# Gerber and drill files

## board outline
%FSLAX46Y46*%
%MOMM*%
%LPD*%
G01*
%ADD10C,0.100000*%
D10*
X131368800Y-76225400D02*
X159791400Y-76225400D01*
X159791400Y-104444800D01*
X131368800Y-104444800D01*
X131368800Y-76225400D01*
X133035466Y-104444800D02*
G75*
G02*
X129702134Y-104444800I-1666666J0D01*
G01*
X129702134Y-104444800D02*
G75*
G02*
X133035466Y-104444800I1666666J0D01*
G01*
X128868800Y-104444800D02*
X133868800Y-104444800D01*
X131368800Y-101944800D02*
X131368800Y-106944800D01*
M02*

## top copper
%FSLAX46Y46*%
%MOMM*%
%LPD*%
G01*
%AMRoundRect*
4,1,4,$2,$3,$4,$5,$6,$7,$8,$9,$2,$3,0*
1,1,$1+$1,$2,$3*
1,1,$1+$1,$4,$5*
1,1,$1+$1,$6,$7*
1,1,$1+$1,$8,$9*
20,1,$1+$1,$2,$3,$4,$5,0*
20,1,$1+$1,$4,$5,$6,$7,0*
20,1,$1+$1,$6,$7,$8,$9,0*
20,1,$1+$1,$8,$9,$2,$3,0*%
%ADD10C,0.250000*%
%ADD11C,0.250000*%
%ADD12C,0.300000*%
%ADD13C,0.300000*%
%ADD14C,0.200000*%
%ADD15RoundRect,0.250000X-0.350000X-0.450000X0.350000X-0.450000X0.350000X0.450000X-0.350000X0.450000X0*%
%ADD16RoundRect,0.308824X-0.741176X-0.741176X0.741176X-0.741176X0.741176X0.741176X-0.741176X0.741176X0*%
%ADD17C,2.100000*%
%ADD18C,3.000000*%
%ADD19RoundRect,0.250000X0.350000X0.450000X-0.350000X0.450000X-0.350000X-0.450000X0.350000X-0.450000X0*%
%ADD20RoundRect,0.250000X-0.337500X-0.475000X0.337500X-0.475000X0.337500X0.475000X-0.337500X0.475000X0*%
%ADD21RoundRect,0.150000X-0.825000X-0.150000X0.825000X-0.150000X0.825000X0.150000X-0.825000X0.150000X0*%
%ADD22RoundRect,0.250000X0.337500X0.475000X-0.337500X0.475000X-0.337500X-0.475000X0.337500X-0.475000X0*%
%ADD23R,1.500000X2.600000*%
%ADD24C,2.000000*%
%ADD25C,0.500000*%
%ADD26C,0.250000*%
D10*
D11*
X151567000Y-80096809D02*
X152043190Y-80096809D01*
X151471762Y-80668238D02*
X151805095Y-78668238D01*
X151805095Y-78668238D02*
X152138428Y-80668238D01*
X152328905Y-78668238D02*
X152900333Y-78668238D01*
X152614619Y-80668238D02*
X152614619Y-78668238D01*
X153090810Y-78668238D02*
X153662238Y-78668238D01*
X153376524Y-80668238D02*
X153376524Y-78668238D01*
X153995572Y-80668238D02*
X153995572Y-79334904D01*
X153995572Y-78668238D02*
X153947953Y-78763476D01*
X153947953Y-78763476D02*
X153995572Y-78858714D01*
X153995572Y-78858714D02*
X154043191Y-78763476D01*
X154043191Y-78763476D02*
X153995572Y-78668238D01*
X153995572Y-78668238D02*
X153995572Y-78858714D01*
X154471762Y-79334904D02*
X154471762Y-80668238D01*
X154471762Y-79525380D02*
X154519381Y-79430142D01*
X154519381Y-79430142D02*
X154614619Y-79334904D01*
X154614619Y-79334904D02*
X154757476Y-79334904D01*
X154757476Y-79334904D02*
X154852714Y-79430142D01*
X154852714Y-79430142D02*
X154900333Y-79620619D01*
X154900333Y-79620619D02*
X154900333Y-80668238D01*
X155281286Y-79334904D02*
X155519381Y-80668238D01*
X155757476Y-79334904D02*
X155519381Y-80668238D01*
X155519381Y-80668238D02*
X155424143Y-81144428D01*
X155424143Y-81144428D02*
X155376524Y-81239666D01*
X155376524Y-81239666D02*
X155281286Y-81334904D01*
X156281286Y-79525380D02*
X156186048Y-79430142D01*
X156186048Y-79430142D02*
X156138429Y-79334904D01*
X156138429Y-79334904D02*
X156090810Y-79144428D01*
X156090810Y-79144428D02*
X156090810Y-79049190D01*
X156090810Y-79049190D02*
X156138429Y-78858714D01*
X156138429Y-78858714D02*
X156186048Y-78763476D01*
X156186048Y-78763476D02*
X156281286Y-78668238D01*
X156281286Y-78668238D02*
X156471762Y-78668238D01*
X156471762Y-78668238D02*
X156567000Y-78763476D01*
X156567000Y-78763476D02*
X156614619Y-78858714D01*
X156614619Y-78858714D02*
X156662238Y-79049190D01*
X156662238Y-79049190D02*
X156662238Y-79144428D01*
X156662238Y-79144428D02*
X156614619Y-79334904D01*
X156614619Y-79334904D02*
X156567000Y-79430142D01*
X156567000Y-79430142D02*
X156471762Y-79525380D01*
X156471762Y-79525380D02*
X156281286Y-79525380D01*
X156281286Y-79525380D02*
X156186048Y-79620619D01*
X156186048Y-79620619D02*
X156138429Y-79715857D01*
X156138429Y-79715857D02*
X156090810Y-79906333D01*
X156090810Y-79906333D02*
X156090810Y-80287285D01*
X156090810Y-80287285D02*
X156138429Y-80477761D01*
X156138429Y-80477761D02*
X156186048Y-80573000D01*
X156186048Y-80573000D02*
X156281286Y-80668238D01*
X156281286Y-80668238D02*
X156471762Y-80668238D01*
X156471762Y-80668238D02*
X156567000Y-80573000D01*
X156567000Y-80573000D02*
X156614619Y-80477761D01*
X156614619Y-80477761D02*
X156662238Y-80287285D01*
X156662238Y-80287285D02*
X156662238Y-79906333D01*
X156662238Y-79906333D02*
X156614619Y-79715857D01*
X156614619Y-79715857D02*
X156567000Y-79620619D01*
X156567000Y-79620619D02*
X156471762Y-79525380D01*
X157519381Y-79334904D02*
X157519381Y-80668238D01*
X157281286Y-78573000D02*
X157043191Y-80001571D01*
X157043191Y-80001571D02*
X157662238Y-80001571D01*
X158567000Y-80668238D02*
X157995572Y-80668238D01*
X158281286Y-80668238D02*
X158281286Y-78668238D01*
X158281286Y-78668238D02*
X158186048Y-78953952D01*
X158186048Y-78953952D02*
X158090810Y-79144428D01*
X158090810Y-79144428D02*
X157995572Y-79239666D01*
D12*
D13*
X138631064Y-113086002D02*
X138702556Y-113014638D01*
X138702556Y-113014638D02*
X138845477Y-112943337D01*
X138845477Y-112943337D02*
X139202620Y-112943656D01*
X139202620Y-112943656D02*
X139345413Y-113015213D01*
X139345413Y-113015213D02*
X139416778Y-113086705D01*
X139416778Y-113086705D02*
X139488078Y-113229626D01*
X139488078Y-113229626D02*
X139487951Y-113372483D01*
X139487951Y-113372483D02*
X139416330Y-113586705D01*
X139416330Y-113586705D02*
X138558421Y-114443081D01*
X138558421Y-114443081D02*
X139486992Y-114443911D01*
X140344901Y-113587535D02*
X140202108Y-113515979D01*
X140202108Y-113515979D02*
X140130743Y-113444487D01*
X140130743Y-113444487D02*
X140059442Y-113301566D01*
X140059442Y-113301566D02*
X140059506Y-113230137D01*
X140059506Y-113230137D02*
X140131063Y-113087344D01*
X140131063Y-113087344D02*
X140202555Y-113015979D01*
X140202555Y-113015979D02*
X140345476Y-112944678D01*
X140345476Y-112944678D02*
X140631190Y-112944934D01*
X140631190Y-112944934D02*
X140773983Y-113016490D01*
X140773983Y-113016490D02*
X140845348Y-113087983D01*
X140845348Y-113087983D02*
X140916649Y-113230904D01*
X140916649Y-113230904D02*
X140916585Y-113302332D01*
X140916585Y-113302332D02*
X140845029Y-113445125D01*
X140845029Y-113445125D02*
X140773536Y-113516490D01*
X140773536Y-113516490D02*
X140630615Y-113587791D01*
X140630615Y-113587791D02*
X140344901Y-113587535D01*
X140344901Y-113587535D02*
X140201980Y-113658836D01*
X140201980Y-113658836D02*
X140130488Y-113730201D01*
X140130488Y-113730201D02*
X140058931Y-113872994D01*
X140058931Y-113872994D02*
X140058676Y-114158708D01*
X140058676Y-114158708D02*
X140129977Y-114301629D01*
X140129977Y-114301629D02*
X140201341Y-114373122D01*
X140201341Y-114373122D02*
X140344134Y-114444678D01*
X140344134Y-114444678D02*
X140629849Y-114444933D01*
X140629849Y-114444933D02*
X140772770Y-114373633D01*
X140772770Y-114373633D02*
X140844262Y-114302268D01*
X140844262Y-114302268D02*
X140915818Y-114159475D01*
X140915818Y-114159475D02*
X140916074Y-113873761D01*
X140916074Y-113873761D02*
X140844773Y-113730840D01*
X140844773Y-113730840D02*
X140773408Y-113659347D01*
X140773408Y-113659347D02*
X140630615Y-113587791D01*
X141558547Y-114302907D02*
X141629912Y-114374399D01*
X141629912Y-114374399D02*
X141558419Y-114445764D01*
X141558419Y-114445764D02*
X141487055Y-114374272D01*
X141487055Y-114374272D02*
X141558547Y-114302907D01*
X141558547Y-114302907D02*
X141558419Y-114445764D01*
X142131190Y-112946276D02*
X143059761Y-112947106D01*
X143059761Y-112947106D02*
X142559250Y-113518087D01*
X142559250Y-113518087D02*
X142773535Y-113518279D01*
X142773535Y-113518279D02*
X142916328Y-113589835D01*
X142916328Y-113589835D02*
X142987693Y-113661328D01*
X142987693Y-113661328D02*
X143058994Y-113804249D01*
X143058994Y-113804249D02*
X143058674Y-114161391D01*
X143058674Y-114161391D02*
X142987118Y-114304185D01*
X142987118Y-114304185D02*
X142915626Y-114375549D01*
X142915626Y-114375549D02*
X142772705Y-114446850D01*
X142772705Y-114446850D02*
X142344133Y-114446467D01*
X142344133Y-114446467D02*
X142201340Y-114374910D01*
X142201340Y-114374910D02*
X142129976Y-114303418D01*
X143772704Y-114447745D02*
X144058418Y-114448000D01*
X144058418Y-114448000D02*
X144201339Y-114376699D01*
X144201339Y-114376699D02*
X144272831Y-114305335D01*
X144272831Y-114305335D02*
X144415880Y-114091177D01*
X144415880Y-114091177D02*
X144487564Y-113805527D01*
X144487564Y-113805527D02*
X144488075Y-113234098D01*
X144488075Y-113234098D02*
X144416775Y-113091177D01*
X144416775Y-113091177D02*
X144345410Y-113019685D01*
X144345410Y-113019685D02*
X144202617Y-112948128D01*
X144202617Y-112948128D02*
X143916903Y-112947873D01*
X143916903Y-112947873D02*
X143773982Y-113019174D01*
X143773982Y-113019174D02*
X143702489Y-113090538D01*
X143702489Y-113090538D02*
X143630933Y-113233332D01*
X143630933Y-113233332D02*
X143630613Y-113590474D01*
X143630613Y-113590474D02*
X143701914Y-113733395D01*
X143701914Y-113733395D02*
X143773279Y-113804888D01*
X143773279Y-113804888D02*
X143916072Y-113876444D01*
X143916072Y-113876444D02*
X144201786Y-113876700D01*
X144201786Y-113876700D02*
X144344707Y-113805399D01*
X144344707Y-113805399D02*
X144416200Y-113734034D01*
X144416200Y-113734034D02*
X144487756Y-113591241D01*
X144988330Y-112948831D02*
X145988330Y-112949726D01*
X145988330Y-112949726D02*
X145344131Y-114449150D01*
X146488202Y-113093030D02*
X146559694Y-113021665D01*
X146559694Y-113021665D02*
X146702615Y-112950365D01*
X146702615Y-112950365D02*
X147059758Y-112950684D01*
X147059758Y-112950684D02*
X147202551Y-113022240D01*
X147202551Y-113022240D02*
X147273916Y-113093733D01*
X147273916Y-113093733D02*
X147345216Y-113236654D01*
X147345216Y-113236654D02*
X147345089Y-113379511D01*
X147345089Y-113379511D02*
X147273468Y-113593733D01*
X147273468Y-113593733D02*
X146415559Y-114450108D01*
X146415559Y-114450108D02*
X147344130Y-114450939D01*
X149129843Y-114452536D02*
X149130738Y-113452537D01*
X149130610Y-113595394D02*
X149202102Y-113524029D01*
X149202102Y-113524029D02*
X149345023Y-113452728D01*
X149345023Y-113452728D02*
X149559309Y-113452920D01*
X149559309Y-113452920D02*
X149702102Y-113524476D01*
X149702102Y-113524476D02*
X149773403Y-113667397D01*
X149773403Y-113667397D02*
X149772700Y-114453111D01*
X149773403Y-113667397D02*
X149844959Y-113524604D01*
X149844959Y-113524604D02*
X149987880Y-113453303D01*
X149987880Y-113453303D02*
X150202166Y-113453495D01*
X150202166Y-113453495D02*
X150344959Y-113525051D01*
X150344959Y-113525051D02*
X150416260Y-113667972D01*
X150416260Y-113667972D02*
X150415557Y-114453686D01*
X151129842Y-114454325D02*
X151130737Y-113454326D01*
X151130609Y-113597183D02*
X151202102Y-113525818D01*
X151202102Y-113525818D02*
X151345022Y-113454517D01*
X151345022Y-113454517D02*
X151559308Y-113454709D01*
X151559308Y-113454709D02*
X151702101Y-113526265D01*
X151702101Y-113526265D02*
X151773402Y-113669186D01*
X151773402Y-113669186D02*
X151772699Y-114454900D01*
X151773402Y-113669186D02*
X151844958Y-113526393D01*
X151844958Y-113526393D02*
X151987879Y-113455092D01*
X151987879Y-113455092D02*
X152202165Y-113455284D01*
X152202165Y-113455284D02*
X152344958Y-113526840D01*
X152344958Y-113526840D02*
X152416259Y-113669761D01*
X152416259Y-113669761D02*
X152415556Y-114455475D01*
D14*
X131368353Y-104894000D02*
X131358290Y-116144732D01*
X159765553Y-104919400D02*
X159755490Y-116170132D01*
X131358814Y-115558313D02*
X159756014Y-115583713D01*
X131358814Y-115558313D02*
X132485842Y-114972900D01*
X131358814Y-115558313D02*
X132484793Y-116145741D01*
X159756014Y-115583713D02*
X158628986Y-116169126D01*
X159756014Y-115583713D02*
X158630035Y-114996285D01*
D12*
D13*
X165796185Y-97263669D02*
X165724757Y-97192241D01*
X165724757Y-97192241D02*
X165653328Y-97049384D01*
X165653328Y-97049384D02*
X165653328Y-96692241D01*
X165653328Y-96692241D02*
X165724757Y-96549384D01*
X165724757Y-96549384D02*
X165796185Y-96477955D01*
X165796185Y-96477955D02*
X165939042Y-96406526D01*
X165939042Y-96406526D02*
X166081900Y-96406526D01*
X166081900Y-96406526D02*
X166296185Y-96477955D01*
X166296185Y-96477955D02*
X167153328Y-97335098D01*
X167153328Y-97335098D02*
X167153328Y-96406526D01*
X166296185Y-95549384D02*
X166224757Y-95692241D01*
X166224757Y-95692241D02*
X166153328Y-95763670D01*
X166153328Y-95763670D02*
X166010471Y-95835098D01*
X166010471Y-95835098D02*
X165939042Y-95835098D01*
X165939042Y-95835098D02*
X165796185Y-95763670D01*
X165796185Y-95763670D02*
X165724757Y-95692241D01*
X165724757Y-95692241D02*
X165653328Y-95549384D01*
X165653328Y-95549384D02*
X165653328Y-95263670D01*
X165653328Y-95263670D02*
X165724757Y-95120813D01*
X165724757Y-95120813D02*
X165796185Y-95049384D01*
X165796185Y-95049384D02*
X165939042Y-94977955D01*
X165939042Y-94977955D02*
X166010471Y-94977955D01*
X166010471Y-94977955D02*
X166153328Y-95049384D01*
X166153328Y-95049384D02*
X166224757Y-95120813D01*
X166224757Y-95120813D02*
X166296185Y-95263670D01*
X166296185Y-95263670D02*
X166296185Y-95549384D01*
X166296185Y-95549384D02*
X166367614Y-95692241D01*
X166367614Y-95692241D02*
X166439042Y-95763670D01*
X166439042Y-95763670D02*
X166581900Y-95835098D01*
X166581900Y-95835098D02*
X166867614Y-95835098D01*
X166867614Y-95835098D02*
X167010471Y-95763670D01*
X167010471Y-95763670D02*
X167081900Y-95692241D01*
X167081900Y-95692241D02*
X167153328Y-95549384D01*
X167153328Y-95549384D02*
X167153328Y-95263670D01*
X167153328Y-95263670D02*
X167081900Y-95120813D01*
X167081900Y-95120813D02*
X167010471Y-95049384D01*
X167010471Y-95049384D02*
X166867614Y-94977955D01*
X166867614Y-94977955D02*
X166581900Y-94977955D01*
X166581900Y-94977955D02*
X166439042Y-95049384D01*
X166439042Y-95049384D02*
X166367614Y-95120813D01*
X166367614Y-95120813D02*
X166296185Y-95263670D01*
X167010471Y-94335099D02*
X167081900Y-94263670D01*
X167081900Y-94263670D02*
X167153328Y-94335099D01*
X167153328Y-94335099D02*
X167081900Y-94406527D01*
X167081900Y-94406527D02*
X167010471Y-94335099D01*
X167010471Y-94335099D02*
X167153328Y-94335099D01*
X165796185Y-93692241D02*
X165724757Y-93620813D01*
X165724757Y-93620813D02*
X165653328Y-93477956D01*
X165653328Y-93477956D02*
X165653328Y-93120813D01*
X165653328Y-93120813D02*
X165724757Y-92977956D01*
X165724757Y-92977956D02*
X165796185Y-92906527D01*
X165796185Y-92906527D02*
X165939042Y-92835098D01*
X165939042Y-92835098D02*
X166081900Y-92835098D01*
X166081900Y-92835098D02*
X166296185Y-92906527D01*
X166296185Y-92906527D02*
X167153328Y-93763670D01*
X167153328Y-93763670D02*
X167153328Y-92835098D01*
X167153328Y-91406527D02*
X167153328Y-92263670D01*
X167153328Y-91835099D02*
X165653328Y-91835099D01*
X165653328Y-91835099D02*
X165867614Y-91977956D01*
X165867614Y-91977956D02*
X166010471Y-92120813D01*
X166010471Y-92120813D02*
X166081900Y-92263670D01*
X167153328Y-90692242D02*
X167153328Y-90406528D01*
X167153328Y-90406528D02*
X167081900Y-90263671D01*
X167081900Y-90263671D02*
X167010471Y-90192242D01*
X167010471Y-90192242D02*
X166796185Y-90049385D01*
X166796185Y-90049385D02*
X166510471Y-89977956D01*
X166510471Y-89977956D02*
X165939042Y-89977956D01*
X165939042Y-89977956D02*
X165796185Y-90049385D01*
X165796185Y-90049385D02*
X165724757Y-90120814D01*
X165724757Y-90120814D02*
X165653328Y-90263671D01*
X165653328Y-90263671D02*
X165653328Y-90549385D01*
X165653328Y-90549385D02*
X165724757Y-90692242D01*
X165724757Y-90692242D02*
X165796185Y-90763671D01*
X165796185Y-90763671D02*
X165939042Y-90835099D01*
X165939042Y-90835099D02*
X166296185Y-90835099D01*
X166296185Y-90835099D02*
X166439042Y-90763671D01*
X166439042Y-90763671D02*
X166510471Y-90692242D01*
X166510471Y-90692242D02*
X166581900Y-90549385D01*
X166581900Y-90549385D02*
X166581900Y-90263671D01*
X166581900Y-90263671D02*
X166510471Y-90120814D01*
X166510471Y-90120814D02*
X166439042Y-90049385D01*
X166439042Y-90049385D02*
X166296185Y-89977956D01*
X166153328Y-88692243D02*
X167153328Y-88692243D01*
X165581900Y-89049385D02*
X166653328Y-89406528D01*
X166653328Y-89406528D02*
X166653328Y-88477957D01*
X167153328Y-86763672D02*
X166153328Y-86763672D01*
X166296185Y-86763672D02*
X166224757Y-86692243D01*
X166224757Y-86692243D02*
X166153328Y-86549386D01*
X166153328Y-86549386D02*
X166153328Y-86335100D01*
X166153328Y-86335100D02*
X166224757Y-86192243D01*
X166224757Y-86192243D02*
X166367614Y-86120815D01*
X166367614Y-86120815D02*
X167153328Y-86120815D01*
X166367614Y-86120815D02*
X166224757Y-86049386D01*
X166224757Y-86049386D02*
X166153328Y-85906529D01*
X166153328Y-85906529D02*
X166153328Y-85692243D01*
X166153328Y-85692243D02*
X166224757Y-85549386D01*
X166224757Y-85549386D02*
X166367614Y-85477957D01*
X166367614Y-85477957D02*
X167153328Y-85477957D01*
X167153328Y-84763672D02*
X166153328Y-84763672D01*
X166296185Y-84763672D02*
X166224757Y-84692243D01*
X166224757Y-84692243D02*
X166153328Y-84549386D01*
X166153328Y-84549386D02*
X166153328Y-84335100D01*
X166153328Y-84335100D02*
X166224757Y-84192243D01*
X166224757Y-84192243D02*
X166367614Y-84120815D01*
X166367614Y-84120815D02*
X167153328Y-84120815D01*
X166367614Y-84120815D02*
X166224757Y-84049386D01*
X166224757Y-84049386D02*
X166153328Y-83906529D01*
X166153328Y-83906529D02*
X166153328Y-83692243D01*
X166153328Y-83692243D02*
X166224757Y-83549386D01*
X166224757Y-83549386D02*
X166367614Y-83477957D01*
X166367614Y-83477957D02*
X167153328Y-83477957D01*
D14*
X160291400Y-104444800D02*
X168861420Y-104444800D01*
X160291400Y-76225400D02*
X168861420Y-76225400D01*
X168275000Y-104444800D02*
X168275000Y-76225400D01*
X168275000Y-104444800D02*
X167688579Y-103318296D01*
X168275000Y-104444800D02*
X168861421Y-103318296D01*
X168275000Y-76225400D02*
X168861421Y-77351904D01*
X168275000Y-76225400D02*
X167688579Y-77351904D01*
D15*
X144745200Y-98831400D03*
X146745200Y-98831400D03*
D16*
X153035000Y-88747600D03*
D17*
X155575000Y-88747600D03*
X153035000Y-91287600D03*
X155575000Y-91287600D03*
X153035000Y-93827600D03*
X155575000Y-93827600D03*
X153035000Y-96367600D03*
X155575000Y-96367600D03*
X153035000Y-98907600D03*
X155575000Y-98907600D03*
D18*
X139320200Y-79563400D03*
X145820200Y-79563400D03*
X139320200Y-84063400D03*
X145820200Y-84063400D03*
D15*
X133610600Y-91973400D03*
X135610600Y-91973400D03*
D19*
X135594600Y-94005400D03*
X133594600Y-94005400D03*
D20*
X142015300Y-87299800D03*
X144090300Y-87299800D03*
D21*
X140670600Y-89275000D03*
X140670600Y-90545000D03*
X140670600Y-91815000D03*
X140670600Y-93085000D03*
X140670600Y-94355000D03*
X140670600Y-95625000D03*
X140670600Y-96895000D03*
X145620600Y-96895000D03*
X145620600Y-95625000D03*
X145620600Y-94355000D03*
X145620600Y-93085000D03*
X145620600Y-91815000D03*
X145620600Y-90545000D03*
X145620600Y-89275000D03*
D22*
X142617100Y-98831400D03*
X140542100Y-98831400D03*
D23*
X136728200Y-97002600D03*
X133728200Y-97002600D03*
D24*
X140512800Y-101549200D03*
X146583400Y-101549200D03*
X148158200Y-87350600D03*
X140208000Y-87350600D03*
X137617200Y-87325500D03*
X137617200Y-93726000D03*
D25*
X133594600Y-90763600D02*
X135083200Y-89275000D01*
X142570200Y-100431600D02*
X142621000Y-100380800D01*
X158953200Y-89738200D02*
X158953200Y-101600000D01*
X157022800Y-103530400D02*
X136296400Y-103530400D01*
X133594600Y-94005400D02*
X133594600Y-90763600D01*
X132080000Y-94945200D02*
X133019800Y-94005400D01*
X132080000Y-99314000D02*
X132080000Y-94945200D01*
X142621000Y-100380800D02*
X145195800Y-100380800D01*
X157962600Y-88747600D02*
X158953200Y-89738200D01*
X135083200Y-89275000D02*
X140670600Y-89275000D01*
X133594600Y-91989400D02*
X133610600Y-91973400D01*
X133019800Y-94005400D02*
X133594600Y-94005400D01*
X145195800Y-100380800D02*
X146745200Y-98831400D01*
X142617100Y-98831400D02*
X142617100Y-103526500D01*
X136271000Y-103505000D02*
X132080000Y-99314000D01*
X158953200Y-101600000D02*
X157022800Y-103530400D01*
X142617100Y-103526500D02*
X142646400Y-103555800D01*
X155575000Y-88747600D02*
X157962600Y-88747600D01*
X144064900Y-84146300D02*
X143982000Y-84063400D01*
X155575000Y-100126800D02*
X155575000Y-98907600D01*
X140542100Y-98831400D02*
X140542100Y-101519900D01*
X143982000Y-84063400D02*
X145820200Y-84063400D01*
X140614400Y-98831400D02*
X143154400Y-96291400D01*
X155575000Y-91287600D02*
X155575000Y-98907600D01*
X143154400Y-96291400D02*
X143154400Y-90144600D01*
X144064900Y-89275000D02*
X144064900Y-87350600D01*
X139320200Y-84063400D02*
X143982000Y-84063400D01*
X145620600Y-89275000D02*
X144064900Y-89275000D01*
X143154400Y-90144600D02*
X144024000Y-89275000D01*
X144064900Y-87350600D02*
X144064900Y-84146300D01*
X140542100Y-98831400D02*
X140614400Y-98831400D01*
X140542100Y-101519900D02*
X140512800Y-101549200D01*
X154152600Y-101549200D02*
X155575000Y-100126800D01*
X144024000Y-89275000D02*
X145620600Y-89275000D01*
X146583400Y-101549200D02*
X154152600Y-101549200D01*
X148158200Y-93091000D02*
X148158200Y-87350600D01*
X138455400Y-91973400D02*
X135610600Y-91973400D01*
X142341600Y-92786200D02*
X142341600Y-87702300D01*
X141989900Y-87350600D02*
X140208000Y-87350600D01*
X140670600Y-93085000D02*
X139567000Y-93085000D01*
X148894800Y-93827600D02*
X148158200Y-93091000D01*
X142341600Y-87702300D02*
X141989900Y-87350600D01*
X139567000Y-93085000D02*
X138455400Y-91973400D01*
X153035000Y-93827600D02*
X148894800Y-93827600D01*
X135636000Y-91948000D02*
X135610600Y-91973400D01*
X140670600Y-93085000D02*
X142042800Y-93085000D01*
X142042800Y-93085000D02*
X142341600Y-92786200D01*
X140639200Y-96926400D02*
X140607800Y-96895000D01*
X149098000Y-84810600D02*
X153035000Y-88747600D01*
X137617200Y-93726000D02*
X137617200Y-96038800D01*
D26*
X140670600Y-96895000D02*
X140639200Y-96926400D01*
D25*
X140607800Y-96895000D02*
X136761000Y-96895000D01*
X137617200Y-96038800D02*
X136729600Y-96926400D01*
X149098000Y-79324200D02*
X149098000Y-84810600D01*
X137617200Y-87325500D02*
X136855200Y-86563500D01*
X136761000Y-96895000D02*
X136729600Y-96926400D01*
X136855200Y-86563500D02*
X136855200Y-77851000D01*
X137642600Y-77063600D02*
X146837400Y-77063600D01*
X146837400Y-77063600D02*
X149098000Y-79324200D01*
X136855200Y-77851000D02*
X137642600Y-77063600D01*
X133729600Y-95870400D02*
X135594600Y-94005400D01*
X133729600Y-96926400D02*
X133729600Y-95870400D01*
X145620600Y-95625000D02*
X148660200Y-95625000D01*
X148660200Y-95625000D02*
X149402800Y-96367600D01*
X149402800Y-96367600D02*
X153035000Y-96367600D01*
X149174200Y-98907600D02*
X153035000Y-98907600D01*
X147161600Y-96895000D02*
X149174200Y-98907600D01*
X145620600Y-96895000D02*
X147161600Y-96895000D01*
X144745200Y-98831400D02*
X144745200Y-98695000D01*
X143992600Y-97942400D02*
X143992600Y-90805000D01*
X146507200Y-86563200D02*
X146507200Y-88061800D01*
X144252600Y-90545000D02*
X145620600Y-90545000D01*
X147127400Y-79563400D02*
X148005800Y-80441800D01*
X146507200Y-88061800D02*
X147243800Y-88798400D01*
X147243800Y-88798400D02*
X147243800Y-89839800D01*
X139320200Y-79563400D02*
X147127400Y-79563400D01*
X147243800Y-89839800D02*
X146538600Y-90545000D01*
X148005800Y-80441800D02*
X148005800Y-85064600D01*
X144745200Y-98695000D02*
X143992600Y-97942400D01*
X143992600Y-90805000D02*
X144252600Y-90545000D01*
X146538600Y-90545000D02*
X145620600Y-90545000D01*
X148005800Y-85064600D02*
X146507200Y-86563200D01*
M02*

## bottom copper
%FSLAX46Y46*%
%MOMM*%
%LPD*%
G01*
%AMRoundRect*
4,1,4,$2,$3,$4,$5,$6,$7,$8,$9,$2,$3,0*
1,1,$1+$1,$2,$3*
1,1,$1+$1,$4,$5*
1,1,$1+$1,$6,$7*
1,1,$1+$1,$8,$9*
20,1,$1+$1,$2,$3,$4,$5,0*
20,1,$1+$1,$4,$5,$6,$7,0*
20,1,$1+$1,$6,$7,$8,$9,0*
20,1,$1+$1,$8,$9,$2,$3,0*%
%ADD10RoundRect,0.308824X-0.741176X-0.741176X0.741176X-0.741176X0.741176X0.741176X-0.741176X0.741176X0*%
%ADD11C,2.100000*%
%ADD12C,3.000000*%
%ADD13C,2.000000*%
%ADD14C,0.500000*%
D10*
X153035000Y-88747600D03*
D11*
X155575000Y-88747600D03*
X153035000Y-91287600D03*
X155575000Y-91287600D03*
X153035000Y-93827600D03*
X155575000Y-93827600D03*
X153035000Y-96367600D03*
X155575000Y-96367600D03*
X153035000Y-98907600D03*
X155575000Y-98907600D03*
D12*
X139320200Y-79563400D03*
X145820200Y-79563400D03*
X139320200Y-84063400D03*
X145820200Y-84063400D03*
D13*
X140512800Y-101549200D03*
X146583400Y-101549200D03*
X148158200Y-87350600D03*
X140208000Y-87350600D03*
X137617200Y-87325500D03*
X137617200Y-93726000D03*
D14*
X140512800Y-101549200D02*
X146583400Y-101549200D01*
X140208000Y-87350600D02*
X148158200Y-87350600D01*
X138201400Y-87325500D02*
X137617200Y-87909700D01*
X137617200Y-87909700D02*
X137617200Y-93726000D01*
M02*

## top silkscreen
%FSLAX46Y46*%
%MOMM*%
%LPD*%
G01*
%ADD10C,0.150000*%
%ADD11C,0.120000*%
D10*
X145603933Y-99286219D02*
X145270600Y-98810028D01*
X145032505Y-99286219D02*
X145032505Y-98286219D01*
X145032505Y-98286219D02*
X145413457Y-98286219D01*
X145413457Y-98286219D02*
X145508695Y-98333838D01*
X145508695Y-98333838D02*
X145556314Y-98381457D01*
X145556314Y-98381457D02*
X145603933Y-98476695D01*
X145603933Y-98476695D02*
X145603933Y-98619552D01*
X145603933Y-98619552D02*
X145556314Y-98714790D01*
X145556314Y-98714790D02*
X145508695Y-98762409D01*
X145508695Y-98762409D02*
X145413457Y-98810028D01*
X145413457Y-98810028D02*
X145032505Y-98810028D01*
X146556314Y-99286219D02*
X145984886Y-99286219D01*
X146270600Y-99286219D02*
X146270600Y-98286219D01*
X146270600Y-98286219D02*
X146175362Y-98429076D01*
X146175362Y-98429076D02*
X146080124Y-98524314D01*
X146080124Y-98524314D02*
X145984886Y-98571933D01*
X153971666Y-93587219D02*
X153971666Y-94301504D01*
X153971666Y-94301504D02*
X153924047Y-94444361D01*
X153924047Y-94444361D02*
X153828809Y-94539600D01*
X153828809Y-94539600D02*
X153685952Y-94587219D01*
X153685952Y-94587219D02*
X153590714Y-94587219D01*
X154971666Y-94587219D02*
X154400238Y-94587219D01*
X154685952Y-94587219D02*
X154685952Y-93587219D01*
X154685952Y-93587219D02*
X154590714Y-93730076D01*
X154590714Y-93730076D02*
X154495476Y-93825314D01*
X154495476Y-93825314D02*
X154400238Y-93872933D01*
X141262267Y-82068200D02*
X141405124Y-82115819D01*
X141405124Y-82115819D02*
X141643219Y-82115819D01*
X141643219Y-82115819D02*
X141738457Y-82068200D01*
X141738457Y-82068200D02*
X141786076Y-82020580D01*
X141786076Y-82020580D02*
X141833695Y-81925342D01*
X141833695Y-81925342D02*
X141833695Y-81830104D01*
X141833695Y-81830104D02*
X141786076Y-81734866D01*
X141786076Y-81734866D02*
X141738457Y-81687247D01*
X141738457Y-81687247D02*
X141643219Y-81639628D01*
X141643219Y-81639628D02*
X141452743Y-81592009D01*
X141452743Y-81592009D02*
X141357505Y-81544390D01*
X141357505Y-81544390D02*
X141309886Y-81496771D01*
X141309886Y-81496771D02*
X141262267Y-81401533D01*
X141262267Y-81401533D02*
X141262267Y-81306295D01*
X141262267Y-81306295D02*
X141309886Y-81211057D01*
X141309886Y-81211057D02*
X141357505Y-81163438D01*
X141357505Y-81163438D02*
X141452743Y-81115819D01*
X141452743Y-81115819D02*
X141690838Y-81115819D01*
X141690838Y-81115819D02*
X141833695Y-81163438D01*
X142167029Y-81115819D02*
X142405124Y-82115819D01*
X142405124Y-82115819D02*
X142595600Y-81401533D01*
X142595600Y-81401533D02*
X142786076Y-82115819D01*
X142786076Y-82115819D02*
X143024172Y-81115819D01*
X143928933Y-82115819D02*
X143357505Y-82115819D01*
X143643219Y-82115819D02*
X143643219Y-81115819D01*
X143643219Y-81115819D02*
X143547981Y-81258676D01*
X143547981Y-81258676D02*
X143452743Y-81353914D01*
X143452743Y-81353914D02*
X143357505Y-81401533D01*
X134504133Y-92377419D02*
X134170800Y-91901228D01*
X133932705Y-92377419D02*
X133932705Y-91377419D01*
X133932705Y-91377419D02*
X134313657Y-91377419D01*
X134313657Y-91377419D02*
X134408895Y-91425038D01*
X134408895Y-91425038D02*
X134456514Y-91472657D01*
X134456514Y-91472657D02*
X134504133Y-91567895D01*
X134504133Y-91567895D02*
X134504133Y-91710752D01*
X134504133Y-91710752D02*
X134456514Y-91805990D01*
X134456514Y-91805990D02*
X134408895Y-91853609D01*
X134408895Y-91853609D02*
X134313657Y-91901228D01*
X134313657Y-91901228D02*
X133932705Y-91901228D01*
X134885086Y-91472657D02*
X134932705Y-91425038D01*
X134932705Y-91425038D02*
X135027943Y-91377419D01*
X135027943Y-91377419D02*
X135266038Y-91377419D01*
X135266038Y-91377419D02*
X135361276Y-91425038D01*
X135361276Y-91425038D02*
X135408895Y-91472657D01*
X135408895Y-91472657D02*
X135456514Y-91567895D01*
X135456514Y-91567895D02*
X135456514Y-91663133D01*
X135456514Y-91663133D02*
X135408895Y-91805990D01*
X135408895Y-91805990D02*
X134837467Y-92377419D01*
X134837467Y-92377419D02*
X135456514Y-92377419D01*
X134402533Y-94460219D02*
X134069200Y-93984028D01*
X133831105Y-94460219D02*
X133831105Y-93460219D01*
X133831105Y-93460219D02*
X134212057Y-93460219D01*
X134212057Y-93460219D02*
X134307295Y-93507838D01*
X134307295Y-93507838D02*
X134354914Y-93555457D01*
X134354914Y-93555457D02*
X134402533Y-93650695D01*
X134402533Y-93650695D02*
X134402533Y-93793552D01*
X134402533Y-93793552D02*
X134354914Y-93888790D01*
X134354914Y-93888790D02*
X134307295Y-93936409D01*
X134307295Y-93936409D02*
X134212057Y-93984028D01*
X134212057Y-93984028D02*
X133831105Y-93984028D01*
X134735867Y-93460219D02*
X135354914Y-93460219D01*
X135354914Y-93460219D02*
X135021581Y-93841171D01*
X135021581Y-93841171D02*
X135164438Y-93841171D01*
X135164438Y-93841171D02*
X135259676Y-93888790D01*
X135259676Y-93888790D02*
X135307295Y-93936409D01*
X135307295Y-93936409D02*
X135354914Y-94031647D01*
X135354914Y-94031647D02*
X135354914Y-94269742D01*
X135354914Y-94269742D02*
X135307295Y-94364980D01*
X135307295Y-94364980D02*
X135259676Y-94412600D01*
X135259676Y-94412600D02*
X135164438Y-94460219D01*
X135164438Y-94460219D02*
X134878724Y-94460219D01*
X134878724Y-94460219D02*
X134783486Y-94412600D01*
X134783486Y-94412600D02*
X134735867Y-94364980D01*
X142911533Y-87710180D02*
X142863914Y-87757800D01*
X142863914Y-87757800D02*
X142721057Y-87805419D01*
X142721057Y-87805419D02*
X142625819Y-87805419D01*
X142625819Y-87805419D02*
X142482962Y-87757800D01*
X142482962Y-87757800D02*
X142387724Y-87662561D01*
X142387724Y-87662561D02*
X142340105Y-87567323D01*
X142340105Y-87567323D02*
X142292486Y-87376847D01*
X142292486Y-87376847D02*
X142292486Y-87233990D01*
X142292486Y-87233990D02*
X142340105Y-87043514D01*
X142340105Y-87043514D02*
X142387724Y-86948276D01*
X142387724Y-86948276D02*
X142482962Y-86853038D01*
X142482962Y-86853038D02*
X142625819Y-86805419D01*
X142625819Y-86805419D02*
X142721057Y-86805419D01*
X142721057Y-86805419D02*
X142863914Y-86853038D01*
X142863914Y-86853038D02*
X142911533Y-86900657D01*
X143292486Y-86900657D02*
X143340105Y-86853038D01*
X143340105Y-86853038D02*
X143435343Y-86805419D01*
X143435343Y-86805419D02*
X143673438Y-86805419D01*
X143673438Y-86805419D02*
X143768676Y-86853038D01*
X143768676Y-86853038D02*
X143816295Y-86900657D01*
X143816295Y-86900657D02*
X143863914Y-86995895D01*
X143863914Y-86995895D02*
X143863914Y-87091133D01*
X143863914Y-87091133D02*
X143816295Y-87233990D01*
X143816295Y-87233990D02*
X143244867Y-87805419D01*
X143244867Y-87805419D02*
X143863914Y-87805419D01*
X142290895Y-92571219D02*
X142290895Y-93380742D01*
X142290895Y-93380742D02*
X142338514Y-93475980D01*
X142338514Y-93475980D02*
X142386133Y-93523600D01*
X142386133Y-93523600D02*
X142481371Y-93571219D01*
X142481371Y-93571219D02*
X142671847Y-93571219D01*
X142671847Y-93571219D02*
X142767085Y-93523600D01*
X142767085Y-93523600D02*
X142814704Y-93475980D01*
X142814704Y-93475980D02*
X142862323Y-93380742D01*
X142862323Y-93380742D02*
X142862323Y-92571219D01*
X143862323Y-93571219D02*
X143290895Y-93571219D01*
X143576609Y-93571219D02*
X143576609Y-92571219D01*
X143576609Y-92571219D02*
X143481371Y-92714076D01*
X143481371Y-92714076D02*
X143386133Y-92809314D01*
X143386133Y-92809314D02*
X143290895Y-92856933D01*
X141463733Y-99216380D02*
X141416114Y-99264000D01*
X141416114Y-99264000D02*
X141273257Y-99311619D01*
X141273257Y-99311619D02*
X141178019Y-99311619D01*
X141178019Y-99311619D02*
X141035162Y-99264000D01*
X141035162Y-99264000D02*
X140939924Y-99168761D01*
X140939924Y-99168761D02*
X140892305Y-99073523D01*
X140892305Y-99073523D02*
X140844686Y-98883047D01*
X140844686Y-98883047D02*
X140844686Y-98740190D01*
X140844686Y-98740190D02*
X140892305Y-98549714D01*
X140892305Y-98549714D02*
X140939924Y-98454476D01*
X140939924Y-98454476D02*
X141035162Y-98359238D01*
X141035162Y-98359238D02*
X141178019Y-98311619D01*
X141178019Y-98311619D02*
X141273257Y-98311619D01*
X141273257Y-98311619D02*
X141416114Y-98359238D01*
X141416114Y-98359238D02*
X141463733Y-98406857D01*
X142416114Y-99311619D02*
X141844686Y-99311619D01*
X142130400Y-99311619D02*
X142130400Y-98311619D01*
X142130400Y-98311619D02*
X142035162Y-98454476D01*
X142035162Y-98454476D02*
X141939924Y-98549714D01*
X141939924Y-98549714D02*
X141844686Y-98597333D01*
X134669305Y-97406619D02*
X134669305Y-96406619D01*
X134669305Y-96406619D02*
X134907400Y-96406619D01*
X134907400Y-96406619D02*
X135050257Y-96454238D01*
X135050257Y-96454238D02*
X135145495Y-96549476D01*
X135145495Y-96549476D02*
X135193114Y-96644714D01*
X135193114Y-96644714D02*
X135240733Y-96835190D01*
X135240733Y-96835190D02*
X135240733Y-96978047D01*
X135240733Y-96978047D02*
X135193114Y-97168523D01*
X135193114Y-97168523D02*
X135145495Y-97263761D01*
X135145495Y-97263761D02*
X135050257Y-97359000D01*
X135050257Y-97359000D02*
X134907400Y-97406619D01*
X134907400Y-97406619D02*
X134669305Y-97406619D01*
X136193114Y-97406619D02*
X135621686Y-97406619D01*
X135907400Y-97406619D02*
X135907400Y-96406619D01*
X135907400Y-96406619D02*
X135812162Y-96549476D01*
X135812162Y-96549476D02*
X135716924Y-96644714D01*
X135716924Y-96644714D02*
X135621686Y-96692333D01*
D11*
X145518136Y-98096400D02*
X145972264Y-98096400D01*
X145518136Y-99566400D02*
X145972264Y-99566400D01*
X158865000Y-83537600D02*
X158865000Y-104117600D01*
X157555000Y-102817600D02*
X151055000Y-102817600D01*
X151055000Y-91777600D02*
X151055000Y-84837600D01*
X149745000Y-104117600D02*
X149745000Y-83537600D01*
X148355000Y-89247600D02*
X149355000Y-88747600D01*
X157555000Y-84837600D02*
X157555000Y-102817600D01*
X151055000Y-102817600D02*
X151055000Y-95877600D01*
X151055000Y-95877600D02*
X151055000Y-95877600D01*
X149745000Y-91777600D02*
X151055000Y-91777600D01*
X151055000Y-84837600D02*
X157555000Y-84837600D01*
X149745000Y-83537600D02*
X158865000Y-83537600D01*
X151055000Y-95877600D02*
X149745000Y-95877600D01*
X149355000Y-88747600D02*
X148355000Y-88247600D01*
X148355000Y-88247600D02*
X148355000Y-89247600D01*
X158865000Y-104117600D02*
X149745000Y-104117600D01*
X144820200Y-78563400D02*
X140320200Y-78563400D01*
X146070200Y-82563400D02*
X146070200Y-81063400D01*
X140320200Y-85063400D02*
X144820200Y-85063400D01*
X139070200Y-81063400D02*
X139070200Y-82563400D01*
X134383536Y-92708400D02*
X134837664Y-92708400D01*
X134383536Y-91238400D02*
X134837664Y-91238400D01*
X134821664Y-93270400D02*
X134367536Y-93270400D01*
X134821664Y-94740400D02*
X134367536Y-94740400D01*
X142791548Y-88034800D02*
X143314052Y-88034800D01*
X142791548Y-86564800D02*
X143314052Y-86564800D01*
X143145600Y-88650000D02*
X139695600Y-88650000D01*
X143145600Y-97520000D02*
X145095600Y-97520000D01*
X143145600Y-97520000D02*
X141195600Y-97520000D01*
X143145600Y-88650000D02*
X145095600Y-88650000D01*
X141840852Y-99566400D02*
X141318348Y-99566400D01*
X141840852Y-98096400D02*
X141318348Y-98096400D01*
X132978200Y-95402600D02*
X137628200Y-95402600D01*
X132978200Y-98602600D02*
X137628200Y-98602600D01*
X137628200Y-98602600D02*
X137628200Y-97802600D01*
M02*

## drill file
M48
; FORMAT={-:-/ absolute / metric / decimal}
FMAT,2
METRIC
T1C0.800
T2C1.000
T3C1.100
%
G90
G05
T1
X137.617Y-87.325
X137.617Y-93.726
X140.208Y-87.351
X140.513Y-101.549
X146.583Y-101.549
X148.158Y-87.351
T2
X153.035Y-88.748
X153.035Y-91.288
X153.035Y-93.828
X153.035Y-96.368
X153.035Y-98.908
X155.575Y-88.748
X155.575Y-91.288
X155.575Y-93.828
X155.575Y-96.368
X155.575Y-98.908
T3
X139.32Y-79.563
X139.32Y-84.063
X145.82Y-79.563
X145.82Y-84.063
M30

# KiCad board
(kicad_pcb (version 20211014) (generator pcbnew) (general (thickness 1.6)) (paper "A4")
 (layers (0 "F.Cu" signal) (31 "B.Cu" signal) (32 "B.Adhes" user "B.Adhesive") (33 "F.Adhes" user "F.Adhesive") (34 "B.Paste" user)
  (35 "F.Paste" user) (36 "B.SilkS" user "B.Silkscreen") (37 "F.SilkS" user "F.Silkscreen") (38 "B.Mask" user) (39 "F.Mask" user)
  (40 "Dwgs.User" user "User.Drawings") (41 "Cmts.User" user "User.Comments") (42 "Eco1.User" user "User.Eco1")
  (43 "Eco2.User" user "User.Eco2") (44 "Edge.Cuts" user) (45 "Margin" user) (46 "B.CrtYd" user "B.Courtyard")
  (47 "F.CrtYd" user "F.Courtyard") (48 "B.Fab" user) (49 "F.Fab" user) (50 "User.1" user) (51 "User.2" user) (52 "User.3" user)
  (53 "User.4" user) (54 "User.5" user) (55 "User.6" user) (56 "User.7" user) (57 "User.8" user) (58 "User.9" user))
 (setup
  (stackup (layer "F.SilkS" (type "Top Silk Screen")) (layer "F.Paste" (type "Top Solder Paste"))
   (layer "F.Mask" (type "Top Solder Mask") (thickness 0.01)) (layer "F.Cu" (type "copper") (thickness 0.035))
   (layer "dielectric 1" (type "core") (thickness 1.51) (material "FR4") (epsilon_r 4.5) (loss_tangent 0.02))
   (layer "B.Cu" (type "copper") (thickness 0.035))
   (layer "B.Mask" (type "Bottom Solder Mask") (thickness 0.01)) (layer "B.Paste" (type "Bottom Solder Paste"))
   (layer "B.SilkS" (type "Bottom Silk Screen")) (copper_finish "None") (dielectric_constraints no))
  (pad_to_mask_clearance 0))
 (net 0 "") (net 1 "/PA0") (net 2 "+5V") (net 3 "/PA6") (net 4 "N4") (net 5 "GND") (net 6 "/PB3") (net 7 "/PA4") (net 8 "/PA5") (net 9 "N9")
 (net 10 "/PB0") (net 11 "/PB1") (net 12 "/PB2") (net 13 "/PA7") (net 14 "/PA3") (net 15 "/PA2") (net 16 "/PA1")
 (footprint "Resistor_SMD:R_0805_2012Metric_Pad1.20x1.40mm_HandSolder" (layer "F.Cu") (at 145.7452 98.8314)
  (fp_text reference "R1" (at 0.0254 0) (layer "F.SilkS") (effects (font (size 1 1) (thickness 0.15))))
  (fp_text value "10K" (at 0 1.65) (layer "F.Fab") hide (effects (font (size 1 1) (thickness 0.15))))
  (fp_line (start -0.227064 -0.735) (end 0.227064 -0.735) (layer "F.SilkS") (width 0.12))
  (fp_line (start -0.227064 0.735) (end 0.227064 0.735) (layer "F.SilkS") (width 0.12))
  (pad "1" smd roundrect locked (at -1 0) (size 1.2 1.4) (layers "F.Cu" "F.Paste" "F.Mask") (roundrect_rratio 0.2083333333) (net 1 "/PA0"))
  (pad "2" smd roundrect locked (at 1 0) (size 1.2 1.4) (layers "F.Cu" "F.Paste" "F.Mask") (roundrect_rratio 0.2083333333) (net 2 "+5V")))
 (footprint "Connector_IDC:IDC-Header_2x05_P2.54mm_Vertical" (layer "F.Cu") (at 153.035 88.7476)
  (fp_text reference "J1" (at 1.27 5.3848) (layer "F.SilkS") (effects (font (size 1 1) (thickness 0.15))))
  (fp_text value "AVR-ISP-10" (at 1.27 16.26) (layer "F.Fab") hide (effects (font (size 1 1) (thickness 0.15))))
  (fp_line (start 5.83 -5.21) (end 5.83 15.37) (layer "F.SilkS") (width 0.12))
  (fp_line (start 4.52 14.07) (end -1.98 14.07) (layer "F.SilkS") (width 0.12))
  (fp_line (start -1.98 3.03) (end -1.98 -3.91) (layer "F.SilkS") (width 0.12))
  (fp_line (start -3.29 15.37) (end -3.29 -5.21) (layer "F.SilkS") (width 0.12))
  (fp_line (start -4.68 0.5) (end -3.68 0) (layer "F.SilkS") (width 0.12))
  (fp_line (start 4.52 -3.91) (end 4.52 14.07) (layer "F.SilkS") (width 0.12))
  (fp_line (start -1.98 14.07) (end -1.98 7.13) (layer "F.SilkS") (width 0.12))
  (fp_line (start -1.98 7.13) (end -1.98 7.13) (layer "F.SilkS") (width 0.12))
  (fp_line (start -3.29 3.03) (end -1.98 3.03) (layer "F.SilkS") (width 0.12))
  (fp_line (start -1.98 -3.91) (end 4.52 -3.91) (layer "F.SilkS") (width 0.12))
  (fp_line (start -3.29 -5.21) (end 5.83 -5.21) (layer "F.SilkS") (width 0.12))
  (fp_line (start -1.98 7.13) (end -3.29 7.13) (layer "F.SilkS") (width 0.12))
  (fp_line (start -3.68 0) (end -4.68 -0.5) (layer "F.SilkS") (width 0.12))
  (fp_line (start -4.68 -0.5) (end -4.68 0.5) (layer "F.SilkS") (width 0.12))
  (fp_line (start 5.83 15.37) (end -3.29 15.37) (layer "F.SilkS") (width 0.12))
  (pad "1" thru_hole roundrect locked (at 0 0) (size 2.1 2.1) (drill 1) (layers *.Cu *.Mask) (roundrect_rratio 0.1470590476) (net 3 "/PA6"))
  (pad "2" thru_hole circle locked (at 2.54 0) (size 2.1 2.1) (drill 1) (layers *.Cu *.Mask) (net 2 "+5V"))
  (pad "3" thru_hole circle locked (at 0 2.54) (size 2.1 2.1) (drill 1) (layers *.Cu *.Mask) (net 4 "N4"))
  (pad "4" thru_hole circle locked (at 2.54 2.54) (size 2.1 2.1) (drill 1) (layers *.Cu *.Mask) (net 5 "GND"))
  (pad "5" thru_hole circle locked (at 0 5.08) (size 2.1 2.1) (drill 1) (layers *.Cu *.Mask) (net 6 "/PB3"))
  (pad "6" thru_hole circle locked (at 2.54 5.08) (size 2.1 2.1) (drill 1) (layers *.Cu *.Mask) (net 5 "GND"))
  (pad "7" thru_hole circle locked (at 0 7.62) (size 2.1 2.1) (drill 1) (layers *.Cu *.Mask) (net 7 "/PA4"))
  (pad "8" thru_hole circle locked (at 2.54 7.62) (size 2.1 2.1) (drill 1) (layers *.Cu *.Mask) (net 5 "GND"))
  (pad "9" thru_hole circle locked (at 0 10.16) (size 2.1 2.1) (drill 1) (layers *.Cu *.Mask) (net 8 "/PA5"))
  (pad "10" thru_hole circle locked (at 2.54 10.16) (size 2.1 2.1) (drill 1) (layers *.Cu *.Mask) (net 5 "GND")))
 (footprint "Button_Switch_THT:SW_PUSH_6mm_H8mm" (layer "F.Cu") (at 139.3202 79.5634)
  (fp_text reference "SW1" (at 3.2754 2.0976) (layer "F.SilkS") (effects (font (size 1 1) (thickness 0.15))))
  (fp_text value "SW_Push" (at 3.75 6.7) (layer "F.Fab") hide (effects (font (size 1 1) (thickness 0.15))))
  (fp_line (start 5.5 -1) (end 1 -1) (layer "F.SilkS") (width 0.12))
  (fp_line (start 6.75 3) (end 6.75 1.5) (layer "F.SilkS") (width 0.12))
  (fp_line (start 1 5.5) (end 5.5 5.5) (layer "F.SilkS") (width 0.12))
  (fp_line (start -0.25 1.5) (end -0.25 3) (layer "F.SilkS") (width 0.12))
  (pad "1" thru_hole circle locked (at 0 0 90) (size 3 3) (drill 1.1) (layers *.Cu *.Mask) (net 1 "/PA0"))
  (pad "1" thru_hole circle locked (at 6.5 0 90) (size 3 3) (drill 1.1) (layers *.Cu *.Mask) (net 1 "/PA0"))
  (pad "2" thru_hole circle locked (at 0 4.5 90) (size 3 3) (drill 1.1) (layers *.Cu *.Mask) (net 5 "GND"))
  (pad "2" thru_hole circle locked (at 6.5 4.5 90) (size 3 3) (drill 1.1) (layers *.Cu *.Mask) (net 5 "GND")))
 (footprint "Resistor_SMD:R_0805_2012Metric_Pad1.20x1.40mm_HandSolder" (layer "F.Cu") (at 134.6106 91.9734)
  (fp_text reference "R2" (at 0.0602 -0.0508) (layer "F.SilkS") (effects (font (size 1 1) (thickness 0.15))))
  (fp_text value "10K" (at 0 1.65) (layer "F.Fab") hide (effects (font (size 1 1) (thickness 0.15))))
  (fp_line (start -0.227064 0.735) (end 0.227064 0.735) (layer "F.SilkS") (width 0.12))
  (fp_line (start -0.227064 -0.735) (end 0.227064 -0.735) (layer "F.SilkS") (width 0.12))
  (pad "1" smd roundrect locked (at -1 0) (size 1.2 1.4) (layers "F.Cu" "F.Paste" "F.Mask") (roundrect_rratio 0.2083333333) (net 2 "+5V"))
  (pad "2" smd roundrect locked (at 1 0) (size 1.2 1.4) (layers "F.Cu" "F.Paste" "F.Mask") (roundrect_rratio 0.2083333333) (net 6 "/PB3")))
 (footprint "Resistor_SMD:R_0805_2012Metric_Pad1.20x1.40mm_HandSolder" (layer "F.Cu") (at 134.5946 94.0054 180)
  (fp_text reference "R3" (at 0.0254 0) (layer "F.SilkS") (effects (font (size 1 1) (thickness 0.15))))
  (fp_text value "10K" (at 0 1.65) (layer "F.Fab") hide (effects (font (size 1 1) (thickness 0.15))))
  (fp_line (start -0.227064 0.735) (end 0.227064 0.735) (layer "F.SilkS") (width 0.12))
  (fp_line (start -0.227064 -0.735) (end 0.227064 -0.735) (layer "F.SilkS") (width 0.12))
  (pad "1" smd roundrect locked (at -1 0 180) (size 1.2 1.4) (layers "F.Cu" "F.Paste" "F.Mask") (roundrect_rratio 0.2083333333) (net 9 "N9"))
  (pad "2" smd roundrect locked (at 1 0 180) (size 1.2 1.4) (layers "F.Cu" "F.Paste" "F.Mask") (roundrect_rratio 0.2083333333) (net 2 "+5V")))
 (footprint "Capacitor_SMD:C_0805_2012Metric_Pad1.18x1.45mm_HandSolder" (layer "F.Cu") (at 143.0528 87.2998)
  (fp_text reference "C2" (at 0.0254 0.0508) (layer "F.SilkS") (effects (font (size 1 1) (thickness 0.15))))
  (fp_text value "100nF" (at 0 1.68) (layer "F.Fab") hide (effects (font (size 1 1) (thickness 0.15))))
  (fp_line (start -0.261252 0.735) (end 0.261252 0.735) (layer "F.SilkS") (width 0.12))
  (fp_line (start -0.261252 -0.735) (end 0.261252 -0.735) (layer "F.SilkS") (width 0.12))
  (pad "1" smd roundrect locked (at -1.0375 0) (size 1.175 1.45) (layers "F.Cu" "F.Paste" "F.Mask") (roundrect_rratio 0.2127659574)
   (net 6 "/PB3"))
  (pad "2" smd roundrect locked (at 1.0375 0) (size 1.175 1.45) (layers "F.Cu" "F.Paste" "F.Mask") (roundrect_rratio 0.2127659574)
   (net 5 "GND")))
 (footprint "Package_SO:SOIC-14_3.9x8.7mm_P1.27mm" (layer "F.Cu") (at 143.1456 93.085)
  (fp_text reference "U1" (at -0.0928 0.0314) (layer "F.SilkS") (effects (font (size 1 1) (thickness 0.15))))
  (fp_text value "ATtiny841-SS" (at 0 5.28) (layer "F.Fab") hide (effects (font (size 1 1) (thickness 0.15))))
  (fp_line (start 0 -4.435) (end -3.45 -4.435) (layer "F.SilkS") (width 0.12))
  (fp_line (start 0 4.435) (end 1.95 4.435) (layer "F.SilkS") (width 0.12))
  (fp_line (start 0 4.435) (end -1.95 4.435) (layer "F.SilkS") (width 0.12))
  (fp_line (start 0 -4.435) (end 1.95 -4.435) (layer "F.SilkS") (width 0.12))
  (pad "1" smd roundrect locked (at -2.475 -3.81) (size 1.95 0.6) (layers "F.Cu" "F.Paste" "F.Mask") (roundrect_rratio 0.25) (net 2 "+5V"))
  (pad "2" smd roundrect locked (at -2.475 -2.54) (size 1.95 0.6) (layers "F.Cu" "F.Paste" "F.Mask") (roundrect_rratio 0.25) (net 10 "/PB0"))
  (pad "3" smd roundrect locked (at -2.475 -1.27) (size 1.95 0.6) (layers "F.Cu" "F.Paste" "F.Mask") (roundrect_rratio 0.25) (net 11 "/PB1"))
  (pad "4" smd roundrect locked (at -2.475 0) (size 1.95 0.6) (layers "F.Cu" "F.Paste" "F.Mask") (roundrect_rratio 0.25) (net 6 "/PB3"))
  (pad "5" smd roundrect locked (at -2.475 1.27) (size 1.95 0.6) (layers "F.Cu" "F.Paste" "F.Mask") (roundrect_rratio 0.25) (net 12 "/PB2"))
  (pad "6" smd roundrect locked (at -2.475 2.54) (size 1.95 0.6) (layers "F.Cu" "F.Paste" "F.Mask") (roundrect_rratio 0.25) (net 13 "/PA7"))
  (pad "7" smd roundrect locked (at -2.475 3.81) (size 1.95 0.6) (layers "F.Cu" "F.Paste" "F.Mask") (roundrect_rratio 0.25) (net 3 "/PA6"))
  (pad "8" smd roundrect locked (at 2.475 3.81) (size 1.95 0.6) (layers "F.Cu" "F.Paste" "F.Mask") (roundrect_rratio 0.25) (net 8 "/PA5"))
  (pad "9" smd roundrect locked (at 2.475 2.54) (size 1.95 0.6) (layers "F.Cu" "F.Paste" "F.Mask") (roundrect_rratio 0.25) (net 7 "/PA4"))
  (pad "10" smd roundrect locked (at 2.475 1.27) (size 1.95 0.6) (layers "F.Cu" "F.Paste" "F.Mask") (roundrect_rratio 0.25) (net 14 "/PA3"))
  (pad "11" smd roundrect locked (at 2.475 0) (size 1.95 0.6) (layers "F.Cu" "F.Paste" "F.Mask") (roundrect_rratio 0.25) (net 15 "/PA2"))
  (pad "12" smd roundrect locked (at 2.475 -1.27) (size 1.95 0.6) (layers "F.Cu" "F.Paste" "F.Mask") (roundrect_rratio 0.25) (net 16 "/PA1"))
  (pad "13" smd roundrect locked (at 2.475 -2.54) (size 1.95 0.6) (layers "F.Cu" "F.Paste" "F.Mask") (roundrect_rratio 0.25) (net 1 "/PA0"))
  (pad "14" smd roundrect locked (at 2.475 -3.81) (size 1.95 0.6) (layers "F.Cu" "F.Paste" "F.Mask") (roundrect_rratio 0.25) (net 5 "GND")))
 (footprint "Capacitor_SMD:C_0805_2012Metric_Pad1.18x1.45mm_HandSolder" (layer "F.Cu") (at 141.5796 98.8314 180)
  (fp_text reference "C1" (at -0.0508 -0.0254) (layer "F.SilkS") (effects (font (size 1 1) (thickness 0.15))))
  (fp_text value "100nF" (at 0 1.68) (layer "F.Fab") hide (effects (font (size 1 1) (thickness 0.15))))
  (fp_line (start -0.261252 -0.735) (end 0.261252 -0.735) (layer "F.SilkS") (width 0.12))
  (fp_line (start -0.261252 0.735) (end 0.261252 0.735) (layer "F.SilkS") (width 0.12))
  (pad "1" smd roundrect locked (at -1.0375 0 180) (size 1.175 1.45) (layers "F.Cu" "F.Paste" "F.Mask") (roundrect_rratio 0.2127659574)
   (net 2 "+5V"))
  (pad "2" smd roundrect locked (at 1.0375 0 180) (size 1.175 1.45) (layers "F.Cu" "F.Paste" "F.Mask") (roundrect_rratio 0.2127659574)
   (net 5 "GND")))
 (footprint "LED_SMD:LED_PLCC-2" (layer "F.Cu") (at 135.2282 97.0026 180)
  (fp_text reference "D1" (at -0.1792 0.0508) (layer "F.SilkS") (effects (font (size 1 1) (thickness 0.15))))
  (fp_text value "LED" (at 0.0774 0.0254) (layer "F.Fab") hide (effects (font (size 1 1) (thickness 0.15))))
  (fp_line (start 2.25 1.6) (end -2.4 1.6) (layer "F.SilkS") (width 0.12))
  (fp_line (start 2.25 -1.6) (end -2.4 -1.6) (layer "F.SilkS") (width 0.12))
  (fp_line (start -2.4 -1.6) (end -2.4 -0.8) (layer "F.SilkS") (width 0.12))
  (pad "1" smd rect locked (at -1.5 0 180) (size 1.5 2.6) (layers "F.Cu" "F.Paste" "F.Mask") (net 3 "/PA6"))
  (pad "2" smd rect locked (at 1.5 0 180) (size 1.5 2.6) (layers "F.Cu" "F.Paste" "F.Mask") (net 9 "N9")))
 (gr_rect (start 159.7914 104.4448) (end 131.3688 76.2254) (layer "Edge.Cuts") (width 0.1) (fill none))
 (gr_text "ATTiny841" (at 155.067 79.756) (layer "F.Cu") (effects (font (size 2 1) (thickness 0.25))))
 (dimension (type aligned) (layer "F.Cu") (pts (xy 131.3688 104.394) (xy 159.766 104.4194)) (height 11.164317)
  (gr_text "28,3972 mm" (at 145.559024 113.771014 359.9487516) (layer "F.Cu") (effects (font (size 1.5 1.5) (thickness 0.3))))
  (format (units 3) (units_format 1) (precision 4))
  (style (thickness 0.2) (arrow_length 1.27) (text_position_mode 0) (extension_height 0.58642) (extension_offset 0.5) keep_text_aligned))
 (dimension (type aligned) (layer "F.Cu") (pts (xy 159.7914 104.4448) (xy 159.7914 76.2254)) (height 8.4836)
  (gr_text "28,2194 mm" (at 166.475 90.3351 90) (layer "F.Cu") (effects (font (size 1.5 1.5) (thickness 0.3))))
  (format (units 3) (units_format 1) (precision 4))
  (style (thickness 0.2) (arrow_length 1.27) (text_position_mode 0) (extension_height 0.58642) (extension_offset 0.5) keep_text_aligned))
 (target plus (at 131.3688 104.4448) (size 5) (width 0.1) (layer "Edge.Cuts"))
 (segment (start 133.5946 90.7636) (end 135.0832 89.275) (width 0.5) (layer "F.Cu") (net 2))
 (segment (start 142.5702 100.4316) (end 142.621 100.3808) (width 0.5) (layer "F.Cu") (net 2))
 (segment (start 158.9532 89.7382) (end 158.9532 101.6) (width 0.5) (layer "F.Cu") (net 2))
 (segment (start 157.0228 103.5304) (end 136.2964 103.5304) (width 0.5) (layer "F.Cu") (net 2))
 (segment (start 133.5946 94.0054) (end 133.5946 90.7636) (width 0.5) (layer "F.Cu") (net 2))
 (segment (start 132.08 94.9452) (end 133.0198 94.0054) (width 0.5) (layer "F.Cu") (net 2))
 (segment (start 132.08 99.314) (end 132.08 94.9452) (width 0.5) (layer "F.Cu") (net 2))
 (segment (start 142.621 100.3808) (end 145.1958 100.3808) (width 0.5) (layer "F.Cu") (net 2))
 (segment (start 157.9626 88.7476) (end 158.9532 89.7382) (width 0.5) (layer "F.Cu") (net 2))
 (segment (start 135.0832 89.275) (end 140.6706 89.275) (width 0.5) (layer "F.Cu") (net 2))
 (segment (start 133.5946 91.9894) (end 133.6106 91.9734) (width 0.5) (layer "F.Cu") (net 2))
 (segment (start 133.0198 94.0054) (end 133.5946 94.0054) (width 0.5) (layer "F.Cu") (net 2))
 (segment (start 145.1958 100.3808) (end 146.7452 98.8314) (width 0.5) (layer "F.Cu") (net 2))
 (segment (start 142.6171 98.8314) (end 142.6171 103.5265) (width 0.5) (layer "F.Cu") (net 2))
 (segment (start 136.271 103.505) (end 132.08 99.314) (width 0.5) (layer "F.Cu") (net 2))
 (segment (start 158.9532 101.6) (end 157.0228 103.5304) (width 0.5) (layer "F.Cu") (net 2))
 (segment (start 142.6171 103.5265) (end 142.6464 103.5558) (width 0.5) (layer "F.Cu") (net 2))
 (segment (start 155.575 88.7476) (end 157.9626 88.7476) (width 0.5) (layer "F.Cu") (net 2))
 (segment (start 144.0649 84.1463) (end 143.982 84.0634) (width 0.5) (layer "F.Cu") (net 5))
 (segment (start 155.575 100.1268) (end 155.575 98.9076) (width 0.5) (layer "F.Cu") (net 5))
 (segment (start 140.5421 98.8314) (end 140.5421 101.5199) (width 0.5) (layer "F.Cu") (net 5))
 (segment (start 143.982 84.0634) (end 145.8202 84.0634) (width 0.5) (layer "F.Cu") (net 5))
 (segment (start 140.6144 98.8314) (end 143.1544 96.2914) (width 0.5) (layer "F.Cu") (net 5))
 (segment (start 155.575 91.2876) (end 155.575 98.9076) (width 0.5) (layer "F.Cu") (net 5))
 (segment (start 143.1544 96.2914) (end 143.1544 90.1446) (width 0.5) (layer "F.Cu") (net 5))
 (segment (start 144.0649 89.275) (end 144.0649 87.3506) (width 0.5) (layer "F.Cu") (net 5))
 (segment (start 139.3202 84.0634) (end 143.982 84.0634) (width 0.5) (layer "F.Cu") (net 5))
 (segment (start 145.6206 89.275) (end 144.0649 89.275) (width 0.5) (layer "F.Cu") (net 5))
 (segment (start 143.1544 90.1446) (end 144.024 89.275) (width 0.5) (layer "F.Cu") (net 5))
 (segment (start 144.0649 87.3506) (end 144.0649 84.1463) (width 0.5) (layer "F.Cu") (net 5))
 (segment (start 140.5421 98.8314) (end 140.6144 98.8314) (width 0.5) (layer "F.Cu") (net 5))
 (segment (start 140.5421 101.5199) (end 140.5128 101.5492) (width 0.5) (layer "F.Cu") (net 5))
 (segment (start 154.1526 101.5492) (end 155.575 100.1268) (width 0.5) (layer "F.Cu") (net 5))
 (segment (start 144.024 89.275) (end 145.6206 89.275) (width 0.5) (layer "F.Cu") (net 5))
 (segment (start 146.5834 101.5492) (end 154.1526 101.5492) (width 0.5) (layer "F.Cu") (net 5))
 (via (at 140.5128 101.5492) (size 2) (drill 0.8) (layers "F.Cu" "B.Cu") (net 5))
 (via (at 146.5834 101.5492) (size 2) (drill 0.8) (layers "F.Cu" "B.Cu") (free) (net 5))
 (segment (start 140.5128 101.5492) (end 146.5834 101.5492) (width 0.5) (layer "B.Cu") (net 5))
 (segment (start 148.1582 93.091) (end 148.1582 87.3506) (width 0.5) (layer "F.Cu") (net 6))
 (segment (start 138.4554 91.9734) (end 135.6106 91.9734) (width 0.5) (layer "F.Cu") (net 6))
 (segment (start 142.3416 92.7862) (end 142.3416 87.7023) (width 0.5) (layer "F.Cu") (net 6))
 (segment (start 141.9899 87.3506) (end 140.208 87.3506) (width 0.5) (layer "F.Cu") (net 6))
 (segment (start 140.6706 93.085) (end 139.567 93.085) (width 0.5) (layer "F.Cu") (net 6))
 (segment (start 148.8948 93.8276) (end 148.1582 93.091) (width 0.5) (layer "F.Cu") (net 6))
 (segment (start 142.3416 87.7023) (end 141.9899 87.3506) (width 0.5) (layer "F.Cu") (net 6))
 (segment (start 139.567 93.085) (end 138.4554 91.9734) (width 0.5) (layer "F.Cu") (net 6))
 (segment (start 153.035 93.8276) (end 148.8948 93.8276) (width 0.5) (layer "F.Cu") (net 6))
 (segment (start 135.636 91.948) (end 135.6106 91.9734) (width 0.5) (layer "F.Cu") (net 6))
 (segment (start 140.6706 93.085) (end 142.0428 93.085) (width 0.5) (layer "F.Cu") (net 6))
 (segment (start 142.0428 93.085) (end 142.3416 92.7862) (width 0.5) (layer "F.Cu") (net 6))
 (via (at 148.1582 87.3506) (size 2) (drill 0.8) (layers "F.Cu" "B.Cu") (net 6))
 (via (at 140.208 87.3506) (size 2) (drill 0.8) (layers "F.Cu" "B.Cu") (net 6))
 (segment (start 140.208 87.3506) (end 148.1582 87.3506) (width 0.5) (layer "B.Cu") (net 6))
 (segment (start 140.6392 96.9264) (end 140.6078 96.895) (width 0.5) (layer "F.Cu") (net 3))
 (segment (start 149.098 84.8106) (end 153.035 88.7476) (width 0.5) (layer "F.Cu") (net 3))
 (segment (start 137.6172 93.726) (end 137.6172 96.0388) (width 0.5) (layer "F.Cu") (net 3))
 (segment (start 140.6706 96.895) (end 140.6392 96.9264) (width 0.25) (layer "F.Cu") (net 3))
 (segment (start 140.6078 96.895) (end 136.761 96.895) (width 0.5) (layer "F.Cu") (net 3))
 (segment (start 137.6172 96.0388) (end 136.7296 96.9264) (width 0.5) (layer "F.Cu") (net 3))
 (segment (start 149.098 79.3242) (end 149.098 84.8106) (width 0.5) (layer "F.Cu") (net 3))
 (segment (start 137.6172 87.3255) (end 136.8552 86.5635) (width 0.5) (layer "F.Cu") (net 3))
 (segment (start 136.761 96.895) (end 136.7296 96.9264) (width 0.5) (layer "F.Cu") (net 3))
 (segment (start 136.8552 86.5635) (end 136.8552 77.851) (width 0.5) (layer "F.Cu") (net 3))
 (segment (start 137.6426 77.0636) (end 146.8374 77.0636) (width 0.5) (layer "F.Cu") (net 3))
 (segment (start 146.8374 77.0636) (end 149.098 79.3242) (width 0.5) (layer "F.Cu") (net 3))
 (segment (start 136.8552 77.851) (end 137.6426 77.0636) (width 0.5) (layer "F.Cu") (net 3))
 (via (at 137.6172 87.3255) (size 2) (drill 0.8) (layers "F.Cu" "B.Cu") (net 3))
 (via (at 137.6172 93.726) (size 2) (drill 0.8) (layers "F.Cu" "B.Cu") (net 3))
 (segment (start 138.2014 87.3255) (end 137.6172 87.9097) (width 0.5) (layer "B.Cu") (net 3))
 (segment (start 137.6172 87.9097) (end 137.6172 93.726) (width 0.5) (layer "B.Cu") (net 3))
 (segment (start 133.7296 95.8704) (end 135.5946 94.0054) (width 0.5) (layer "F.Cu") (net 9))
 (segment (start 133.7296 96.9264) (end 133.7296 95.8704) (width 0.5) (layer "F.Cu") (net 9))
 (segment (start 145.6206 95.625) (end 148.6602 95.625) (width 0.5) (layer "F.Cu") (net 7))
 (segment (start 148.6602 95.625) (end 149.4028 96.3676) (width 0.5) (layer "F.Cu") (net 7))
 (segment (start 149.4028 96.3676) (end 153.035 96.3676) (width 0.5) (layer "F.Cu") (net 7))
 (segment (start 149.1742 98.9076) (end 153.035 98.9076) (width 0.5) (layer "F.Cu") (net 8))
 (segment (start 147.1616 96.895) (end 149.1742 98.9076) (width 0.5) (layer "F.Cu") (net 8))
 (segment (start 145.6206 96.895) (end 147.1616 96.895) (width 0.5) (layer "F.Cu") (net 8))
 (segment (start 144.7452 98.8314) (end 144.7452 98.695) (width 0.5) (layer "F.Cu") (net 1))
 (segment (start 143.9926 97.9424) (end 143.9926 90.805) (width 0.5) (layer "F.Cu") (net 1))
 (segment (start 146.5072 86.5632) (end 146.5072 88.0618) (width 0.5) (layer "F.Cu") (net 1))
 (segment (start 144.2526 90.545) (end 145.6206 90.545) (width 0.5) (layer "F.Cu") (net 1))
 (segment (start 147.1274 79.5634) (end 148.0058 80.4418) (width 0.5) (layer "F.Cu") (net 1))
 (segment (start 146.5072 88.0618) (end 147.2438 88.7984) (width 0.5) (layer "F.Cu") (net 1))
 (segment (start 147.2438 88.7984) (end 147.2438 89.8398) (width 0.5) (layer "F.Cu") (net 1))
 (segment (start 139.3202 79.5634) (end 147.1274 79.5634) (width 0.5) (layer "F.Cu") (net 1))
 (segment (start 147.2438 89.8398) (end 146.5386 90.545) (width 0.5) (layer "F.Cu") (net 1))
 (segment (start 148.0058 80.4418) (end 148.0058 85.0646) (width 0.5) (layer "F.Cu") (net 1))
 (segment (start 144.7452 98.695) (end 143.9926 97.9424) (width 0.5) (layer "F.Cu") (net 1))
 (segment (start 143.9926 90.805) (end 144.2526 90.545) (width 0.5) (layer "F.Cu") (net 1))
 (segment (start 146.5386 90.545) (end 145.6206 90.545) (width 0.5) (layer "F.Cu") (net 1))
 (segment (start 148.0058 85.0646) (end 146.5072 86.5632) (width 0.5) (layer "F.Cu") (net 1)))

